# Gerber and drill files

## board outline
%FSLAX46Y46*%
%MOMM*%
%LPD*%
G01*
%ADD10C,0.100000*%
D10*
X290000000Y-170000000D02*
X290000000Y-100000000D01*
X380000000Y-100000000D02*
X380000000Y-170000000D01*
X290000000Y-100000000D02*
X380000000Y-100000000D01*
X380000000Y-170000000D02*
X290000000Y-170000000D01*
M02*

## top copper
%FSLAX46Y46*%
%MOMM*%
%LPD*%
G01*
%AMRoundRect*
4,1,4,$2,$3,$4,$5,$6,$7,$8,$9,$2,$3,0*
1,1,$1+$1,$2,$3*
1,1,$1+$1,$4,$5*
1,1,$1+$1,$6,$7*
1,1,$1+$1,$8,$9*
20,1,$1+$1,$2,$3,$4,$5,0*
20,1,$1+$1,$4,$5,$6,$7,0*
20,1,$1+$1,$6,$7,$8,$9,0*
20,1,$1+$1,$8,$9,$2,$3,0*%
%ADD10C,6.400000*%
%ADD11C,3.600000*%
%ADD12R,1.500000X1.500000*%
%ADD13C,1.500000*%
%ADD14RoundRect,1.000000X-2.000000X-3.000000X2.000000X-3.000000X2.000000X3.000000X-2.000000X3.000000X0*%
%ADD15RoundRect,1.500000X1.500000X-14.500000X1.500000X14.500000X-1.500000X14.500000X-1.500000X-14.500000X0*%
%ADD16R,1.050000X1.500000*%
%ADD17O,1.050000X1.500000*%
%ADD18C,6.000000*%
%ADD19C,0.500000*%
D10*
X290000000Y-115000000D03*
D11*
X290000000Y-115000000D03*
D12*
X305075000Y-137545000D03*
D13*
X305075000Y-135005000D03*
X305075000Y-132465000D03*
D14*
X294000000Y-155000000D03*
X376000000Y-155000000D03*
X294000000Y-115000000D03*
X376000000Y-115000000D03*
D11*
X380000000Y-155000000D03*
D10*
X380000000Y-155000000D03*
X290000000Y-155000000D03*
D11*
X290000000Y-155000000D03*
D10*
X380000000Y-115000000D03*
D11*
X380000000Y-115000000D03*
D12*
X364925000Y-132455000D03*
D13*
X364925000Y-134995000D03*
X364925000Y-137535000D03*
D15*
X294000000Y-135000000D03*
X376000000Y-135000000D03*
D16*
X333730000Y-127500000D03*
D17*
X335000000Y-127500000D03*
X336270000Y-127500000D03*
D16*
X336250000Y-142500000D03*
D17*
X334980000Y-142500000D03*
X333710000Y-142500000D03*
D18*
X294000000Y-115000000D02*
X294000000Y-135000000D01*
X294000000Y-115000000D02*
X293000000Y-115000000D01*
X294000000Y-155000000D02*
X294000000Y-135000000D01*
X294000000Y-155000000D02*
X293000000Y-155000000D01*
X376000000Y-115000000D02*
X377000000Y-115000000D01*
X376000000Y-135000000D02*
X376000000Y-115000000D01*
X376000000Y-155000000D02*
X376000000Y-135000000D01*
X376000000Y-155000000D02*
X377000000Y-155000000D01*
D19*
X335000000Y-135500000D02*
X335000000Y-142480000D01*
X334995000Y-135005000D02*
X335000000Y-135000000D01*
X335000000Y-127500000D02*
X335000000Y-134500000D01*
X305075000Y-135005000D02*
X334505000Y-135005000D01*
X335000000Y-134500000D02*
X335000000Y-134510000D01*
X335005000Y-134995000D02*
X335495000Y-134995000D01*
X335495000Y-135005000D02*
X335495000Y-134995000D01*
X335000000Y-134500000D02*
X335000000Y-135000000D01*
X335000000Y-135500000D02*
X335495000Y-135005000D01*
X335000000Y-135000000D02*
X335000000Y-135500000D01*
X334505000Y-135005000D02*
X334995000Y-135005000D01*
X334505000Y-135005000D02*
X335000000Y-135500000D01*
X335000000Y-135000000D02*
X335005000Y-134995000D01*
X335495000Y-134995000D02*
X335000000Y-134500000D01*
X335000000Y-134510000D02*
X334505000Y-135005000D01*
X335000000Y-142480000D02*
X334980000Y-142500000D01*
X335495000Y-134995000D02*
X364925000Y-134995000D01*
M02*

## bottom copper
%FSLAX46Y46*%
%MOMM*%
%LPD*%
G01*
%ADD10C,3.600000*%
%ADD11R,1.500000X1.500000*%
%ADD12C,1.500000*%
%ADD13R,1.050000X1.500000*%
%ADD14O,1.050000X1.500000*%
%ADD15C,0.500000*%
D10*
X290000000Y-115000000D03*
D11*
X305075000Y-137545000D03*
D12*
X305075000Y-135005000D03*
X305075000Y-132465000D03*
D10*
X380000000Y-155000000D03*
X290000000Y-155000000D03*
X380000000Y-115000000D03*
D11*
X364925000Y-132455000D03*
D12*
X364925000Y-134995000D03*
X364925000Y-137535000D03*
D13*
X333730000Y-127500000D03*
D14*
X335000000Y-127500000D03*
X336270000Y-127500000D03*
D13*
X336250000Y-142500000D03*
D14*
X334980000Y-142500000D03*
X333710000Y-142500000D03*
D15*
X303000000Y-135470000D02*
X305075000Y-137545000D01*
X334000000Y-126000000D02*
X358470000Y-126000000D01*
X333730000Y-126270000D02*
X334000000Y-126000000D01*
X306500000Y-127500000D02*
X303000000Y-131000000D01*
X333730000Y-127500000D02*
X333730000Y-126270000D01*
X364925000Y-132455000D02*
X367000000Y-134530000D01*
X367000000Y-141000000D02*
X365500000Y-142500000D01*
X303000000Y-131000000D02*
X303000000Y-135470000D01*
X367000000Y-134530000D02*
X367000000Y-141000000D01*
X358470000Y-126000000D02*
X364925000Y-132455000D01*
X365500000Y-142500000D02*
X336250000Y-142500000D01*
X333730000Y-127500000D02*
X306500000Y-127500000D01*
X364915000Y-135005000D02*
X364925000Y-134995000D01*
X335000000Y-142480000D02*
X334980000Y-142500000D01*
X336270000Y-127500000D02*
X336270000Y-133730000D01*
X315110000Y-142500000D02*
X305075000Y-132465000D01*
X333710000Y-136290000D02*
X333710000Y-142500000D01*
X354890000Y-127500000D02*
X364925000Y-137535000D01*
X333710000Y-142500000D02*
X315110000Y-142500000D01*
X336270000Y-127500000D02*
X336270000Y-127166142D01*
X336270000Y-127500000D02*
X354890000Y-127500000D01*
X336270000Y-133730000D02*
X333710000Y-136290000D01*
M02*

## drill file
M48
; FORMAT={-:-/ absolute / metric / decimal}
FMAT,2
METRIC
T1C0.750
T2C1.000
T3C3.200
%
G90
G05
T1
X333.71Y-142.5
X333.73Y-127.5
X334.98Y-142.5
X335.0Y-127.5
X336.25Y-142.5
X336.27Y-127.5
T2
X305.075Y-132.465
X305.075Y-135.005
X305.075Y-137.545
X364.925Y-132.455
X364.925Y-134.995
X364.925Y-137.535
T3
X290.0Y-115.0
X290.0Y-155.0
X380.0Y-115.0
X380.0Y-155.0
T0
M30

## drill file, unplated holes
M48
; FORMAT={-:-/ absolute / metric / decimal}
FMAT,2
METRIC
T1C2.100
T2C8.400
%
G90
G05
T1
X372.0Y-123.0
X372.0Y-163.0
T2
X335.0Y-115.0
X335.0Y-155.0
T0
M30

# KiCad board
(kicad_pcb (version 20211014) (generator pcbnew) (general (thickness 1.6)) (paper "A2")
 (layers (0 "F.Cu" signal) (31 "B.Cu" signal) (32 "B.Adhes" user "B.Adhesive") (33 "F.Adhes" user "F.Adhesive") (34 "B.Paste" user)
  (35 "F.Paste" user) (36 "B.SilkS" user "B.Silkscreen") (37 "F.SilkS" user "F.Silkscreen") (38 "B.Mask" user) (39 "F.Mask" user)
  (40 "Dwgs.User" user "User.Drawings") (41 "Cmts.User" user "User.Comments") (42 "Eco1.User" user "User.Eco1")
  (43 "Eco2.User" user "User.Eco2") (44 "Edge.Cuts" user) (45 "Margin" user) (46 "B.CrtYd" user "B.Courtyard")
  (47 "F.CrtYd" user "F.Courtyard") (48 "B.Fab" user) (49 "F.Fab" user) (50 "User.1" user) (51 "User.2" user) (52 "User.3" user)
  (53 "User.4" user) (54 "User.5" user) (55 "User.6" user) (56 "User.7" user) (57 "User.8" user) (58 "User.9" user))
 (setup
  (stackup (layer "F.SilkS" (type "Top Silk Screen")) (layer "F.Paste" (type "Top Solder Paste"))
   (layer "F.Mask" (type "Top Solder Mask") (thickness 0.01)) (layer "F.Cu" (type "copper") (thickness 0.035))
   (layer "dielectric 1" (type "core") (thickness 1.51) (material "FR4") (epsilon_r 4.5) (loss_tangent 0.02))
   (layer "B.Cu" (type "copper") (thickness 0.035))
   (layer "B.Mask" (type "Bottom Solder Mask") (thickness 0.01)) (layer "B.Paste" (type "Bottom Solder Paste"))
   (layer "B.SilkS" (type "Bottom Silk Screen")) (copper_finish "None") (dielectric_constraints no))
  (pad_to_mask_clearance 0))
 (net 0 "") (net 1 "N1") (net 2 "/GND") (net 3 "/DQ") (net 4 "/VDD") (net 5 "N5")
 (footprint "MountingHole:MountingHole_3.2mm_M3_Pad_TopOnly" (layer "F.Cu") (at 290 115)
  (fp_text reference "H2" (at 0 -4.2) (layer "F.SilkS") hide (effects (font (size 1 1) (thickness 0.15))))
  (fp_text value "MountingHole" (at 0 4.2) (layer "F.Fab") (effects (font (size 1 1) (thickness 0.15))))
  (pad "1" connect circle (at 0 0) (size 6.4 6.4) (layers "F.Cu" "F.Mask") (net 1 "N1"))
  (pad "1" thru_hole circle (at 0 0) (size 3.6 3.6) (drill 3.2) (layers *.Cu *.Mask) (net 1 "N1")))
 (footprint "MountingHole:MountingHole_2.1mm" (layer "F.Cu") (at 372 163)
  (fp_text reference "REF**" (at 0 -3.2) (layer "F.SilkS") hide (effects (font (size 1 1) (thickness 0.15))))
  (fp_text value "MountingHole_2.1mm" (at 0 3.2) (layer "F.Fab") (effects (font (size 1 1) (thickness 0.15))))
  (pad "" np_thru_hole circle (at 0 0) (size 2.1 2.1) (drill 2.1) (layers *.Cu *.Mask)))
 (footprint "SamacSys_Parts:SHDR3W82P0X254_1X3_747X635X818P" (layer "F.Cu") (at 305.075 137.545 90)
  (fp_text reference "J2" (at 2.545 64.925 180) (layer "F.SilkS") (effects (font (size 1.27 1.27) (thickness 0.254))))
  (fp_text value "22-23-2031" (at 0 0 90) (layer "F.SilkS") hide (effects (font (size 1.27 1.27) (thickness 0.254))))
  (pad "1" thru_hole rect locked (at 0 0 90) (size 1.5 1.5) (drill 1) (layers *.Cu *.Mask) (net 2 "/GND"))
  (pad "2" thru_hole circle locked (at 2.54 0 90) (size 1.5 1.5) (drill 1) (layers *.Cu *.Mask) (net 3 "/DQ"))
  (pad "3" thru_hole circle locked (at 5.08 0 90) (size 1.5 1.5) (drill 1) (layers *.Cu *.Mask) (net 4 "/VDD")))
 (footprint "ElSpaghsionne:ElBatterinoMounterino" (layer "F.Cu") (at 335 155)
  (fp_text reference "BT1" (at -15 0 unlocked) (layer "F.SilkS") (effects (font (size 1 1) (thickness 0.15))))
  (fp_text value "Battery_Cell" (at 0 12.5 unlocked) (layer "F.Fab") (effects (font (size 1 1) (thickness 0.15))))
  (pad "1" smd roundrect (at -41 0) (size 6 8) (layers "F.Cu" "F.Paste" "F.Mask") (roundrect_rratio 0.1666666667) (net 1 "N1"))
  (pad "2" smd roundrect (at 41 0) (size 6 8) (layers "F.Cu" "F.Paste" "F.Mask") (roundrect_rratio 0.1666666667) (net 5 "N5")))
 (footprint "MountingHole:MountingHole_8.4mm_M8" (layer "F.Cu") (at 335 155)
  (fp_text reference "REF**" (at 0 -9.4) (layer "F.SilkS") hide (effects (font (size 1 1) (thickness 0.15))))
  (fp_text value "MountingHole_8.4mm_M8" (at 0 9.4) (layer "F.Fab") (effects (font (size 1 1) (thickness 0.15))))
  (pad "" np_thru_hole circle (at 0 0) (size 8.4 8.4) (drill 8.4) (layers *.Cu *.Mask)))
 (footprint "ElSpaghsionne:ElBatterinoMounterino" (layer "F.Cu") (at 335 115)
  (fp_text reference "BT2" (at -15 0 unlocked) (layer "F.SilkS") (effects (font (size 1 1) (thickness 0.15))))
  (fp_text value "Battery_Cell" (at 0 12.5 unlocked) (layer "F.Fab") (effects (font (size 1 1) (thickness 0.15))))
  (pad "1" smd roundrect (at -41 0) (size 6 8) (layers "F.Cu" "F.Paste" "F.Mask") (roundrect_rratio 0.1666666667) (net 1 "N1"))
  (pad "2" smd roundrect (at 41 0) (size 6 8) (layers "F.Cu" "F.Paste" "F.Mask") (roundrect_rratio 0.1666666667) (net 5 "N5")))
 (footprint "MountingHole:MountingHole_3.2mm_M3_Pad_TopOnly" (layer "F.Cu") (at 380 155)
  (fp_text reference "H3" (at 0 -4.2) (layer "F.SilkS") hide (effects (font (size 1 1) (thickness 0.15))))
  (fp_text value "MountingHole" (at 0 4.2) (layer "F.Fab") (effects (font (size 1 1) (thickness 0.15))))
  (pad "1" thru_hole circle (at 0 0) (size 3.6 3.6) (drill 3.2) (layers *.Cu *.Mask) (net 5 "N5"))
  (pad "1" connect circle (at 0 0) (size 6.4 6.4) (layers "F.Cu" "F.Mask") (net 5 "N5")))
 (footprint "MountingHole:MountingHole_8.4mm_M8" (layer "F.Cu") (at 335 115)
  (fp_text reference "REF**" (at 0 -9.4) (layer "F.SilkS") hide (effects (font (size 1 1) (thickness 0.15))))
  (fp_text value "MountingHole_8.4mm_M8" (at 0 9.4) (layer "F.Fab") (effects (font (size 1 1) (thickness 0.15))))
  (pad "" np_thru_hole circle (at 0 0) (size 8.4 8.4) (drill 8.4) (layers *.Cu *.Mask)))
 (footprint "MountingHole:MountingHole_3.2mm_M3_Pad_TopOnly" (layer "F.Cu") (at 290 155)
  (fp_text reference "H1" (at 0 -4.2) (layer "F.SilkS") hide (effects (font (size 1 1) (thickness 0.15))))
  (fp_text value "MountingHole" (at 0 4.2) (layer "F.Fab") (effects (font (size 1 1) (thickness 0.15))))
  (pad "1" connect circle (at 0 0) (size 6.4 6.4) (layers "F.Cu" "F.Mask") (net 1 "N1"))
  (pad "1" thru_hole circle (at 0 0) (size 3.6 3.6) (drill 3.2) (layers *.Cu *.Mask) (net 1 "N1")))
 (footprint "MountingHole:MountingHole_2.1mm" (layer "F.Cu") (at 372 123)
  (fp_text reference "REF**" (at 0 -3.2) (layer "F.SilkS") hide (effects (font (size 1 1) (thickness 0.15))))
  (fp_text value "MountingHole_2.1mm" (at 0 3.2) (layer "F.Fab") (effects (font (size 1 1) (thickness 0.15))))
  (pad "" np_thru_hole circle (at 0 0) (size 2.1 2.1) (drill 2.1) (layers *.Cu *.Mask)))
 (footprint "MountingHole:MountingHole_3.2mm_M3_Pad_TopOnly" (layer "F.Cu") (at 380 115)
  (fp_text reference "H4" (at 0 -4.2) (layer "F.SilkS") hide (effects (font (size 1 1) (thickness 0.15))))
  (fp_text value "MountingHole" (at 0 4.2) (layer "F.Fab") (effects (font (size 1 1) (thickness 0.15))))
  (pad "1" connect circle (at 0 0) (size 6.4 6.4) (layers "F.Cu" "F.Mask") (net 5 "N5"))
  (pad "1" thru_hole circle (at 0 0) (size 3.6 3.6) (drill 3.2) (layers *.Cu *.Mask) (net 5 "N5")))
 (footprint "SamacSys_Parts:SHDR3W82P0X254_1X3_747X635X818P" (layer "F.Cu") (at 364.925 132.455 -90)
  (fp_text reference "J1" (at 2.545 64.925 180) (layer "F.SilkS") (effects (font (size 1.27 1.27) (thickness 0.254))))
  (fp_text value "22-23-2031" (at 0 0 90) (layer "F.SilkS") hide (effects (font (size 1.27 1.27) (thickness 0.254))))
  (pad "1" thru_hole rect locked (at 0 0 270) (size 1.5 1.5) (drill 1) (layers *.Cu *.Mask) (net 2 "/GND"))
  (pad "2" thru_hole circle locked (at 2.54 0 270) (size 1.5 1.5) (drill 1) (layers *.Cu *.Mask) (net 3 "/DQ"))
  (pad "3" thru_hole circle locked (at 5.08 0 270) (size 1.5 1.5) (drill 1) (layers *.Cu *.Mask) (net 4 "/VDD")))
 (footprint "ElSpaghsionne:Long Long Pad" (layer "F.Cu") (at 294 135 90)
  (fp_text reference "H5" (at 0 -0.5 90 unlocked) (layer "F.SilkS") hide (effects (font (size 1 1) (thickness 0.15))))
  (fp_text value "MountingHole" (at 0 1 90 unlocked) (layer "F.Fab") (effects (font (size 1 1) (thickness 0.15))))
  (pad "1" smd roundrect (at 0 0 90) (size 32 6) (layers "F.Cu" "F.Paste" "F.Mask") (roundrect_rratio 0.25) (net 1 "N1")))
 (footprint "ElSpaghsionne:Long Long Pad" (layer "F.Cu") (at 376 135 90)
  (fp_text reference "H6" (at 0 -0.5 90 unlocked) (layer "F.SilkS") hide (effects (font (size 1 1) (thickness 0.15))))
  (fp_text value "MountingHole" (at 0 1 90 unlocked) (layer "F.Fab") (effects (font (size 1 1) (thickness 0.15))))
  (pad "1" smd roundrect (at 0 0 90) (size 32 6) (layers "F.Cu" "F.Paste" "F.Mask") (roundrect_rratio 0.25) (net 5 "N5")))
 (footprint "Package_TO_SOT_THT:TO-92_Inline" (layer "B.Cu") (at 333.73 127.5)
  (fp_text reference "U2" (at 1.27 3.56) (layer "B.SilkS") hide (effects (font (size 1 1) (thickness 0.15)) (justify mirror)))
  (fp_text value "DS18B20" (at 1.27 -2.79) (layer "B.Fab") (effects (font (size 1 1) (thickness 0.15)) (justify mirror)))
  (pad "1" thru_hole rect (at 0 0) (size 1.05 1.5) (drill 0.75) (layers *.Cu *.Mask) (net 2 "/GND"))
  (pad "2" thru_hole oval (at 1.27 0) (size 1.05 1.5) (drill 0.75) (layers *.Cu *.Mask) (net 3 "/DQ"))
  (pad "3" thru_hole oval (at 2.54 0) (size 1.05 1.5) (drill 0.75) (layers *.Cu *.Mask) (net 4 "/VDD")))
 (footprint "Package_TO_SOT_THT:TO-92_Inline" (layer "B.Cu") (at 336.25 142.5 180)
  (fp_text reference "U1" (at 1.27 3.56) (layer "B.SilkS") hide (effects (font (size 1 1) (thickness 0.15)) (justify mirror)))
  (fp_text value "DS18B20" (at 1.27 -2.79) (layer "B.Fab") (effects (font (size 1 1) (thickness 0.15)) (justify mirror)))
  (pad "1" thru_hole rect (at 0 0 180) (size 1.05 1.5) (drill 0.75) (layers *.Cu *.Mask) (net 2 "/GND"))
  (pad "2" thru_hole oval (at 1.27 0 180) (size 1.05 1.5) (drill 0.75) (layers *.Cu *.Mask) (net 3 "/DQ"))
  (pad "3" thru_hole oval (at 2.54 0 180) (size 1.05 1.5) (drill 0.75) (layers *.Cu *.Mask) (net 4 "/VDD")))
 (gr_line (start 290 170) (end 290 100) (layer "Edge.Cuts") (width 0.1))
 (gr_line (start 380 100) (end 380 170) (layer "Edge.Cuts") (width 0.1))
 (gr_line (start 290 100) (end 380 100) (layer "Edge.Cuts") (width 0.1))
 (gr_line (start 380 170) (end 290 170) (layer "Edge.Cuts") (width 0.1))
 (segment (start 294 115) (end 294 135) (width 6) (layer "F.Cu") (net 1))
 (segment (start 294 115) (end 293 115) (width 6) (layer "F.Cu") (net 1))
 (segment (start 294 155) (end 294 135) (width 6) (layer "F.Cu") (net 1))
 (segment (start 294 155) (end 293 155) (width 6) (layer "F.Cu") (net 1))
 (segment (start 376 115) (end 377 115) (width 6) (layer "F.Cu") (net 5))
 (segment (start 376 135) (end 376 115) (width 6) (layer "F.Cu") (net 5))
 (segment (start 376 155) (end 376 135) (width 6) (layer "F.Cu") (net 5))
 (segment (start 376 155) (end 377 155) (width 6) (layer "F.Cu") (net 5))
 (segment (start 303 135.47) (end 305.075 137.545) (width 0.5) (layer "B.Cu") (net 2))
 (segment (start 334 126) (end 358.47 126) (width 0.5) (layer "B.Cu") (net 2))
 (segment (start 333.73 126.27) (end 334 126) (width 0.5) (layer "B.Cu") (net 2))
 (segment (start 306.5 127.5) (end 303 131) (width 0.5) (layer "B.Cu") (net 2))
 (segment (start 333.73 127.5) (end 333.73 126.27) (width 0.5) (layer "B.Cu") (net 2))
 (segment (start 364.925 132.455) (end 367 134.53) (width 0.5) (layer "B.Cu") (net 2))
 (segment (start 367 141) (end 365.5 142.5) (width 0.5) (layer "B.Cu") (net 2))
 (segment (start 303 131) (end 303 135.47) (width 0.5) (layer "B.Cu") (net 2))
 (segment (start 367 134.53) (end 367 141) (width 0.5) (layer "B.Cu") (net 2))
 (segment (start 358.47 126) (end 364.925 132.455) (width 0.5) (layer "B.Cu") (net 2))
 (segment (start 365.5 142.5) (end 336.25 142.5) (width 0.5) (layer "B.Cu") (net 2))
 (segment (start 333.73 127.5) (end 306.5 127.5) (width 0.5) (layer "B.Cu") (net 2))
 (segment (start 335 135.5) (end 335 142.48) (width 0.5) (layer "F.Cu") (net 3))
 (segment (start 334.995 135.005) (end 335 135) (width 0.5) (layer "F.Cu") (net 3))
 (segment (start 335 127.5) (end 335 134.5) (width 0.5) (layer "F.Cu") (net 3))
 (segment (start 305.075 135.005) (end 334.505 135.005) (width 0.5) (layer "F.Cu") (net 3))
 (segment (start 335 134.5) (end 335 134.51) (width 0.5) (layer "F.Cu") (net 3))
 (segment (start 335.005 134.995) (end 335.495 134.995) (width 0.5) (layer "F.Cu") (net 3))
 (segment (start 335.495 135.005) (end 335.495 134.995) (width 0.5) (layer "F.Cu") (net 3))
 (segment (start 335 134.5) (end 335 135) (width 0.5) (layer "F.Cu") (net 3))
 (segment (start 335 135.5) (end 335.495 135.005) (width 0.5) (layer "F.Cu") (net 3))
 (segment (start 335 135) (end 335 135.5) (width 0.5) (layer "F.Cu") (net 3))
 (segment (start 334.505 135.005) (end 334.995 135.005) (width 0.5) (layer "F.Cu") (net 3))
 (segment (start 334.505 135.005) (end 335 135.5) (width 0.5) (layer "F.Cu") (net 3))
 (segment (start 335 135) (end 335.005 134.995) (width 0.5) (layer "F.Cu") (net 3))
 (segment (start 335.495 134.995) (end 335 134.5) (width 0.5) (layer "F.Cu") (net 3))
 (segment (start 335 134.51) (end 334.505 135.005) (width 0.5) (layer "F.Cu") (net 3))
 (segment (start 335 142.48) (end 334.98 142.5) (width 0.5) (layer "F.Cu") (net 3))
 (segment (start 335.495 134.995) (end 364.925 134.995) (width 0.5) (layer "F.Cu") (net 3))
 (segment (start 364.915 135.005) (end 364.925 134.995) (width 0.5) (layer "B.Cu") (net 3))
 (segment (start 335 142.48) (end 334.98 142.5) (width 0.5) (layer "B.Cu") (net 3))
 (segment (start 336.27 127.5) (end 336.27 133.73) (width 0.5) (layer "B.Cu") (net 4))
 (segment (start 315.11 142.5) (end 305.075 132.465) (width 0.5) (layer "B.Cu") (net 4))
 (segment (start 333.71 136.29) (end 333.71 142.5) (width 0.5) (layer "B.Cu") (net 4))
 (segment (start 354.89 127.5) (end 364.925 137.535) (width 0.5) (layer "B.Cu") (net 4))
 (segment (start 333.71 142.5) (end 315.11 142.5) (width 0.5) (layer "B.Cu") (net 4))
 (segment (start 336.27 127.5) (end 336.27 127.166142) (width 0.5) (layer "B.Cu") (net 4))
 (segment (start 336.27 127.5) (end 354.89 127.5) (width 0.5) (layer "B.Cu") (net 4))
 (segment (start 336.27 133.73) (end 333.71 136.29) (width 0.5) (layer "B.Cu") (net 4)))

